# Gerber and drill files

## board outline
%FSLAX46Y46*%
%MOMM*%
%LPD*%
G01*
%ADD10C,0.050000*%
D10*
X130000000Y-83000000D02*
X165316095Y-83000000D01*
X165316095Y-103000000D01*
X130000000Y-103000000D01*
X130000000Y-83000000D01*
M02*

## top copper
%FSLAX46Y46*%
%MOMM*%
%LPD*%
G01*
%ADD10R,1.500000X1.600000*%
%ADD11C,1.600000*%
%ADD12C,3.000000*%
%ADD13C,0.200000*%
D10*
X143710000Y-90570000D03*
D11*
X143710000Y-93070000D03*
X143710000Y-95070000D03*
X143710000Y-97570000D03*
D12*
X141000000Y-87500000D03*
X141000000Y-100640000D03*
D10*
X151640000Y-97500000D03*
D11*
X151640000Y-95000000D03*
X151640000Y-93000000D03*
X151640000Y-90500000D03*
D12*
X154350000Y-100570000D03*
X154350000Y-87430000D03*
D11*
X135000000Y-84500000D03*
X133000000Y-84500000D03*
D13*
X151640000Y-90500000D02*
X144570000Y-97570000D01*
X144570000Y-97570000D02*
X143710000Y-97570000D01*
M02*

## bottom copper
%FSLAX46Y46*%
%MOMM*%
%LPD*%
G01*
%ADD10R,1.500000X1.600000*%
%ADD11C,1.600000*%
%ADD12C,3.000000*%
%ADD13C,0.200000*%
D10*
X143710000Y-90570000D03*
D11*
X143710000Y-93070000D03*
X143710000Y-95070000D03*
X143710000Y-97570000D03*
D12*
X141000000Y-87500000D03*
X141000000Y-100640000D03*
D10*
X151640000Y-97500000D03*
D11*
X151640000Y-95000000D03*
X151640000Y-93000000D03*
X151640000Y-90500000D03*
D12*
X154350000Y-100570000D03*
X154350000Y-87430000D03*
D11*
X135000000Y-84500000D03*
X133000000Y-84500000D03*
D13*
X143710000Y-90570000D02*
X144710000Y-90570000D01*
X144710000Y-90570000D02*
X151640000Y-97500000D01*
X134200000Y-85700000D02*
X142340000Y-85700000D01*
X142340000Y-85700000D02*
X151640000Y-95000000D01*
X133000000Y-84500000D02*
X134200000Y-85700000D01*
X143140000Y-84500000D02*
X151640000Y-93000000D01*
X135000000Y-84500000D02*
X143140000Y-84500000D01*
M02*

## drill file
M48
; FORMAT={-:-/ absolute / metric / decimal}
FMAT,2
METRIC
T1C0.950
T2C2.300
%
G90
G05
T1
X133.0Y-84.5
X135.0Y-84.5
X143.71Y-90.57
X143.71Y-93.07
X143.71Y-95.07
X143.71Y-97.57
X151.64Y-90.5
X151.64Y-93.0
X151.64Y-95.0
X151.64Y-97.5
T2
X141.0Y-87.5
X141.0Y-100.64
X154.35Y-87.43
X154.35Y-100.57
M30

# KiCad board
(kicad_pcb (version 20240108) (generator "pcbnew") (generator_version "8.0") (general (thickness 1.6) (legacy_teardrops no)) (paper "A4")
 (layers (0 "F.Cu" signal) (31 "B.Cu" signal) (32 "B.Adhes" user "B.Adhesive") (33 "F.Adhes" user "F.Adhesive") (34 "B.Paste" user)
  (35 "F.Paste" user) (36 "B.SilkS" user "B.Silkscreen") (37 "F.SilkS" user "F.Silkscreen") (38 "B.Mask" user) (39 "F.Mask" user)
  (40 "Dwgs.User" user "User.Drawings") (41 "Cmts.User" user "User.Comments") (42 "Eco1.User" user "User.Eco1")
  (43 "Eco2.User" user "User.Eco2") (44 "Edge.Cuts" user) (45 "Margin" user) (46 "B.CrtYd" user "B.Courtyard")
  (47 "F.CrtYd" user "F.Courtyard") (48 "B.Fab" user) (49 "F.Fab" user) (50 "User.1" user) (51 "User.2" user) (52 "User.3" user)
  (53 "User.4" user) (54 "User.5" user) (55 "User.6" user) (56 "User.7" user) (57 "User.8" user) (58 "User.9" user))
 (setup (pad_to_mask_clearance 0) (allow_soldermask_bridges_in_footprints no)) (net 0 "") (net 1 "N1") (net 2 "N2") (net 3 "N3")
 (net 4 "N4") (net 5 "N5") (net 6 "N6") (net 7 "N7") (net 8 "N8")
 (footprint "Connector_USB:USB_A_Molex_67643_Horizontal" (layer "F.Cu") (at 143.71 90.57 -90)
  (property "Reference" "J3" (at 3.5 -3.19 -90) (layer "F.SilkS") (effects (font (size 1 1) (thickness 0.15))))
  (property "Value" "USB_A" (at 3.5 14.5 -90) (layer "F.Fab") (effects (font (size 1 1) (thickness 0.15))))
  (pad "1" thru_hole rect (at 0 0 270) (size 1.6 1.5) (drill 0.95) (layers "*.Cu" "*.Mask") (remove_unused_layers no) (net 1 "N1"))
  (pad "2" thru_hole circle (at 2.5 0 270) (size 1.6 1.6) (drill 0.95) (layers "*.Cu" "*.Mask") (remove_unused_layers no) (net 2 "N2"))
  (pad "3" thru_hole circle (at 4.5 0 270) (size 1.6 1.6) (drill 0.95) (layers "*.Cu" "*.Mask") (remove_unused_layers no) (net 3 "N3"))
  (pad "4" thru_hole circle (at 7 0 270) (size 1.6 1.6) (drill 0.95) (layers "*.Cu" "*.Mask") (remove_unused_layers no) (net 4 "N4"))
  (pad "5" thru_hole circle (at -3.07 2.71 270) (size 3 3) (drill 2.3) (layers "*.Cu" "*.Mask") (remove_unused_layers no) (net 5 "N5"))
  (pad "5" thru_hole circle (at 10.07 2.71 270) (size 3 3) (drill 2.3) (layers "*.Cu" "*.Mask") (remove_unused_layers no) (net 5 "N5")))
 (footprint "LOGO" (layer "F.Cu") (at 160 84.5)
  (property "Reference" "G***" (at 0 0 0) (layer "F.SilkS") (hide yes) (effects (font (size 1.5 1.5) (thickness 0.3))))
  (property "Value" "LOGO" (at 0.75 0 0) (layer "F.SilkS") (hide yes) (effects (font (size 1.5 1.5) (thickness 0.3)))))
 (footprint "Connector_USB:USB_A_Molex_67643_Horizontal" (layer "F.Cu") (at 151.64 97.5 90)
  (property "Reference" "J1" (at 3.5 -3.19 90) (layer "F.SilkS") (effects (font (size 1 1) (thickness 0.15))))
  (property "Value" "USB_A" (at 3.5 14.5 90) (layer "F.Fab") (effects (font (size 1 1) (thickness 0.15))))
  (pad "1" thru_hole rect (at 0 0 90) (size 1.6 1.5) (drill 0.95) (layers "*.Cu" "*.Mask") (remove_unused_layers no) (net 1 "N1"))
  (pad "2" thru_hole circle (at 2.5 0 90) (size 1.6 1.6) (drill 0.95) (layers "*.Cu" "*.Mask") (remove_unused_layers no) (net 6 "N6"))
  (pad "3" thru_hole circle (at 4.5 0 90) (size 1.6 1.6) (drill 0.95) (layers "*.Cu" "*.Mask") (remove_unused_layers no) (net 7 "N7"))
  (pad "4" thru_hole circle (at 7 0 90) (size 1.6 1.6) (drill 0.95) (layers "*.Cu" "*.Mask") (remove_unused_layers no) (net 4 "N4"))
  (pad "5" thru_hole circle (at -3.07 2.71 90) (size 3 3) (drill 2.3) (layers "*.Cu" "*.Mask") (remove_unused_layers no) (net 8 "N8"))
  (pad "5" thru_hole circle (at 10.07 2.71 90) (size 3 3) (drill 2.3) (layers "*.Cu" "*.Mask") (remove_unused_layers no) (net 8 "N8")))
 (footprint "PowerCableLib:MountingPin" (layer "F.Cu") (at 134 84.5)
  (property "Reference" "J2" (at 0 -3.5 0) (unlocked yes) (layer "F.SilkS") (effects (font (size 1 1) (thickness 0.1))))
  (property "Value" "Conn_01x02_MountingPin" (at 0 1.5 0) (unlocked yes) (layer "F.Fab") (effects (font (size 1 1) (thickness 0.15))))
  (pad "1" thru_hole circle (at 1 0) (size 1.6 1.6) (drill 0.95) (layers "*.Cu" "*.Mask") (remove_unused_layers no) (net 7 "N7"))
  (pad "2" thru_hole circle (at -1 0) (size 1.6 1.6) (drill 0.95) (layers "*.Cu" "*.Mask") (remove_unused_layers no) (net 6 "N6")))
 (gr_rect (start 130 83) (end 165.316095 103) (stroke (width 0.05) (type default)) (fill none) (layer "Edge.Cuts"))
 (segment (start 143.71 90.57) (end 144.71 90.57) (width 0.2) (layer "B.Cu") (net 1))
 (segment (start 144.71 90.57) (end 151.64 97.5) (width 0.2) (layer "B.Cu") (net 1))
 (segment (start 134.2 85.7) (end 142.34 85.7) (width 0.2) (layer "B.Cu") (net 6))
 (segment (start 142.34 85.7) (end 151.64 95) (width 0.2) (layer "B.Cu") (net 6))
 (segment (start 133 84.5) (end 134.2 85.7) (width 0.2) (layer "B.Cu") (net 6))
 (segment (start 151.64 90.5) (end 144.57 97.57) (width 0.2) (layer "F.Cu") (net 4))
 (segment (start 144.57 97.57) (end 143.71 97.57) (width 0.2) (layer "F.Cu") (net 4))
 (segment (start 143.14 84.5) (end 151.64 93) (width 0.2) (layer "B.Cu") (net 7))
 (segment (start 135 84.5) (end 143.14 84.5) (width 0.2) (layer "B.Cu") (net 7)))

